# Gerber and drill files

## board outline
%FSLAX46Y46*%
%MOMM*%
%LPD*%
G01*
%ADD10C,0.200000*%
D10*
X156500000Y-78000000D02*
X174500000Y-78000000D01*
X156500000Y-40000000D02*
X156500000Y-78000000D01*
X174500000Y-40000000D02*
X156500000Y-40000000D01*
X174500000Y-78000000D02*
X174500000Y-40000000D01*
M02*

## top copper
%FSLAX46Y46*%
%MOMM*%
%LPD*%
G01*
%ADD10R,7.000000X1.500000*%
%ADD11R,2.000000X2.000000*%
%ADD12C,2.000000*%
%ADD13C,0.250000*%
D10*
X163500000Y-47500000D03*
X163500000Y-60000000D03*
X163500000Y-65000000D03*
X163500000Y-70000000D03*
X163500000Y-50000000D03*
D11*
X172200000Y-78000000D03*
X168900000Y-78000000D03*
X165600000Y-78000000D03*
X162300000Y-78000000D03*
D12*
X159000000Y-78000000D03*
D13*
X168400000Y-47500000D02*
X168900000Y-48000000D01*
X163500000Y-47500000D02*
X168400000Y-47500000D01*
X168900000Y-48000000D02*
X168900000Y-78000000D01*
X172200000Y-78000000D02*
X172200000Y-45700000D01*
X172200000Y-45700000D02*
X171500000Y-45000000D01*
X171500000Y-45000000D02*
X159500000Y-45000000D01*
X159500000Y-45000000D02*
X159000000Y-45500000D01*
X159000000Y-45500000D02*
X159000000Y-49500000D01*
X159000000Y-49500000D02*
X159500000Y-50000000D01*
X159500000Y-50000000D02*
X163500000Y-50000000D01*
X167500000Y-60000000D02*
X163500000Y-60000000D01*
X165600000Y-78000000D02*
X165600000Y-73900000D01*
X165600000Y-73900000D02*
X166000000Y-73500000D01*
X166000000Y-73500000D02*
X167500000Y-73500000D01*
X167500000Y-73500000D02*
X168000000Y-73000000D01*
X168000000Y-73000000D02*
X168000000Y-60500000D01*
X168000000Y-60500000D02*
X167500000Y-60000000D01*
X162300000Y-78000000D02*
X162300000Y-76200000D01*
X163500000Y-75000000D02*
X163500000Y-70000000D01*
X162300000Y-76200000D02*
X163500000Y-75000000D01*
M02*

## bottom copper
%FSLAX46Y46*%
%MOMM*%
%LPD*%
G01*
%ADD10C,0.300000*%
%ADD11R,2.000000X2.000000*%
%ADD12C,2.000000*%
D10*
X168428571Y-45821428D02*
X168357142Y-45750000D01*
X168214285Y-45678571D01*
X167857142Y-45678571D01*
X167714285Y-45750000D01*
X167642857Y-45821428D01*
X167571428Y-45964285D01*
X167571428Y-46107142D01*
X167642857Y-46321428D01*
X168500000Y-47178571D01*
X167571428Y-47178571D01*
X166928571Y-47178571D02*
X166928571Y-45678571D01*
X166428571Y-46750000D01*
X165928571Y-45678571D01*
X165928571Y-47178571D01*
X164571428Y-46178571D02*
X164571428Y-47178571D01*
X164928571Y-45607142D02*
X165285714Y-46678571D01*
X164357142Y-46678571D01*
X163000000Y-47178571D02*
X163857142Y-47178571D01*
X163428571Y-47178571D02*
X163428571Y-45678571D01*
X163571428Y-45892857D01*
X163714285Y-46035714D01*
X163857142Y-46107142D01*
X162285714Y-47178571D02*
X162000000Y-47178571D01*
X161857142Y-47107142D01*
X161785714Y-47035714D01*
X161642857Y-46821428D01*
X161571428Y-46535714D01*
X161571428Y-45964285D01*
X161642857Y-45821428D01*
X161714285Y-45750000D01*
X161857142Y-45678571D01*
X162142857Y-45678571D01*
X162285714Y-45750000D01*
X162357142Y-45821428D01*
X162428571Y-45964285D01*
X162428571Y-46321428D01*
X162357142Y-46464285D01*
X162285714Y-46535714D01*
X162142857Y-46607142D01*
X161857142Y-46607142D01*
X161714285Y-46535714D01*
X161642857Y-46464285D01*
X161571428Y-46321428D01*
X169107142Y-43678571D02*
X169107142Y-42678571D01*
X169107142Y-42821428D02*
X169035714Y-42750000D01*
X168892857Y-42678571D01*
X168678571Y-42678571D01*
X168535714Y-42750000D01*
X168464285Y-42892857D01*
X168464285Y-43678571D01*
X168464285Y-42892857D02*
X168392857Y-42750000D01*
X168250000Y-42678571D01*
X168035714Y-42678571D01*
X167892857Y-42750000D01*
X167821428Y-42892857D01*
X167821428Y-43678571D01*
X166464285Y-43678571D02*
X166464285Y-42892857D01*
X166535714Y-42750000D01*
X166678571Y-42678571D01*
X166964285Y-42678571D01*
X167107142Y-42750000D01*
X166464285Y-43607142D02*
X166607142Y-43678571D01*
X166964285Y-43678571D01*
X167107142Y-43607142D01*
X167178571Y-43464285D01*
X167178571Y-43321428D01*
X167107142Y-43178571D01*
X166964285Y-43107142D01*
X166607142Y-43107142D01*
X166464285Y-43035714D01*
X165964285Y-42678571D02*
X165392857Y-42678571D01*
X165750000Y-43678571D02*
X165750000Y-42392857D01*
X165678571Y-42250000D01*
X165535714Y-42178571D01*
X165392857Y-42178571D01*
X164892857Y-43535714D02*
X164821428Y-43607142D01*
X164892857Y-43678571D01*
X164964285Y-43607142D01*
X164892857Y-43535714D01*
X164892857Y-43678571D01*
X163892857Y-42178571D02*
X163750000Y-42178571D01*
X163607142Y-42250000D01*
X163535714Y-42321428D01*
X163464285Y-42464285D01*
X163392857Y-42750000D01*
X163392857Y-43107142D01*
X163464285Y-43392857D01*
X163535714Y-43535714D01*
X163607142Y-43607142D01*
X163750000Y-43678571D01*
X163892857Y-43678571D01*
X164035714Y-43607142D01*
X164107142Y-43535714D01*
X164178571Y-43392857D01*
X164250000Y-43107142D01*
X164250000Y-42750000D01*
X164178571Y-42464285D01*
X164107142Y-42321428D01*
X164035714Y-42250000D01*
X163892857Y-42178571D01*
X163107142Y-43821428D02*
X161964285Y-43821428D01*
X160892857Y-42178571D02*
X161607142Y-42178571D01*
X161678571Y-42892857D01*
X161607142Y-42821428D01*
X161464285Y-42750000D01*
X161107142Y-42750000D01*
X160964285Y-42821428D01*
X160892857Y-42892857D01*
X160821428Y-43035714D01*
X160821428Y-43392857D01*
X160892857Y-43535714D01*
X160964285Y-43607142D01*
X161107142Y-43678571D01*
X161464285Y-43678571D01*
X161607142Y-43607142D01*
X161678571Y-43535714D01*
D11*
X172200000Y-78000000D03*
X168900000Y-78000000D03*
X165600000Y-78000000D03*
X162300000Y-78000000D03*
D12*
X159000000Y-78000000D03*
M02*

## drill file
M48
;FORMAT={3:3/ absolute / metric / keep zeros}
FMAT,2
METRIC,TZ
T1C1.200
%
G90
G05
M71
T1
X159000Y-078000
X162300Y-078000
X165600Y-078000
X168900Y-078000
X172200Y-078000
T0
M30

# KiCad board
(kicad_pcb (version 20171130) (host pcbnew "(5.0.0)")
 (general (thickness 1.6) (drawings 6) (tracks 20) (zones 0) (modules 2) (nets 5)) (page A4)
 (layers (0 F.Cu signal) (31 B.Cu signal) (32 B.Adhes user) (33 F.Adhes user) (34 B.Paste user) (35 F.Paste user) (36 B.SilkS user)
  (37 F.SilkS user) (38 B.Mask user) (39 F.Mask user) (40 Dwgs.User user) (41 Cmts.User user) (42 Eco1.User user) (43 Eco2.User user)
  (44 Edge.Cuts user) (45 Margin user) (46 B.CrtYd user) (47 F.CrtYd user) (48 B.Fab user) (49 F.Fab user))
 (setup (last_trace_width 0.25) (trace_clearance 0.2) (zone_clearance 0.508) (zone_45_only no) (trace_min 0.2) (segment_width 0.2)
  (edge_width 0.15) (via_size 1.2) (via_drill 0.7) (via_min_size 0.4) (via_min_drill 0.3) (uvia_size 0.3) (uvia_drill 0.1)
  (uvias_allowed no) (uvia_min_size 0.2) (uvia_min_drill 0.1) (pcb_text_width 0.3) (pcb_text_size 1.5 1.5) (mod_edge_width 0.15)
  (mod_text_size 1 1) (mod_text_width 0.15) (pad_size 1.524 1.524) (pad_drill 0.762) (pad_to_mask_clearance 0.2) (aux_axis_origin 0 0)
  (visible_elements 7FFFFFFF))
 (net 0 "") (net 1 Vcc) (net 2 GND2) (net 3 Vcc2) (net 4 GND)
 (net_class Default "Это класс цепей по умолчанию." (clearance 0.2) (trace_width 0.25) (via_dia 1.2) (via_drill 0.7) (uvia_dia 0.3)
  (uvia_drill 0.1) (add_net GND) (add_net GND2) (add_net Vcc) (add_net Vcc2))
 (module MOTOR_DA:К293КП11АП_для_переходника (layer F.Cu) (at 163.5 86.5)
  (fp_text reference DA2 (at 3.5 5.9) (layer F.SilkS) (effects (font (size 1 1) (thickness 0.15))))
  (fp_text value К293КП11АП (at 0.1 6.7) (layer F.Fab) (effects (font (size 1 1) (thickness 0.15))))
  (pad 11 smd rect (at 0 -39) (size 7 1.5) (layers F.Cu F.Paste F.Mask) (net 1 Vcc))
  (pad 6 smd rect (at 0 -26.5) (size 7 1.5) (layers F.Cu F.Paste F.Mask) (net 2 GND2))
  (pad 4 smd rect (at 0 -21.5) (size 7 1.5) (layers F.Cu F.Paste F.Mask))
  (pad 2 smd rect (at 0 -16.5) (size 7 1.5) (layers F.Cu F.Paste F.Mask) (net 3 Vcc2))
  (pad 10 smd rect (at 0 -36.5) (size 7 1.5) (layers F.Cu F.Paste F.Mask) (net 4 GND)))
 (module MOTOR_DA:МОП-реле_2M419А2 (layer F.Cu) (at 159 78)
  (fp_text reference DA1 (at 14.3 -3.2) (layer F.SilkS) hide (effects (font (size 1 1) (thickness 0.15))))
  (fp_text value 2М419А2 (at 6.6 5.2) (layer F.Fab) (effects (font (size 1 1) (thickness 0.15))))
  (pad 5 thru_hole rect (at 13.2 0) (size 2 2) (drill 1.2) (layers *.Cu *.Paste *.Mask) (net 4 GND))
  (pad 4 thru_hole rect (at 9.9 0) (size 2 2) (drill 1.2) (layers *.Cu *.Paste *.Mask) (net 1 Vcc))
  (pad 3 thru_hole rect (at 6.6 0) (size 2 2) (drill 1.2) (layers *.Cu *.Paste *.Mask) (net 2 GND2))
  (pad 2 thru_hole rect (at 3.3 0) (size 2 2) (drill 1.2) (layers *.Cu *.Paste *.Mask) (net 3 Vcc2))
  (pad 1 thru_hole circle (at 0 0) (size 2 2) (drill 1.2) (layers *.Cu *.Paste *.Mask)))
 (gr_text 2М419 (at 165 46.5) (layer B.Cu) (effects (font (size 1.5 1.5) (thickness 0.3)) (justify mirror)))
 (gr_line (start 156.5 78) (end 174.5 78) (layer Edge.Cuts) (width 0.2))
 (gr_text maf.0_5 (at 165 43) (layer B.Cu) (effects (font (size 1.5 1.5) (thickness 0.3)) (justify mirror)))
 (gr_line (start 156.5 40) (end 156.5 78) (layer Edge.Cuts) (width 0.2))
 (gr_line (start 174.5 40) (end 156.5 40) (layer Edge.Cuts) (width 0.2))
 (gr_line (start 174.5 78) (end 174.5 40) (layer Edge.Cuts) (width 0.2))
 (segment (start 168.4 47.5) (end 168.9 48) (width 0.25) (layer F.Cu) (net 1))
 (segment (start 163.5 47.5) (end 168.4 47.5) (width 0.25) (layer F.Cu) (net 1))
 (segment (start 168.9 48) (end 168.9 78) (width 0.25) (layer F.Cu) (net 1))
 (segment (start 172.2 78) (end 172.2 45.7) (width 0.25) (layer F.Cu) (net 4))
 (segment (start 172.2 45.7) (end 171.5 45) (width 0.25) (layer F.Cu) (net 4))
 (segment (start 171.5 45) (end 159.5 45) (width 0.25) (layer F.Cu) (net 4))
 (segment (start 159.5 45) (end 159 45.5) (width 0.25) (layer F.Cu) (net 4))
 (segment (start 159 45.5) (end 159 49.5) (width 0.25) (layer F.Cu) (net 4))
 (segment (start 159 49.5) (end 159.5 50) (width 0.25) (layer F.Cu) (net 4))
 (segment (start 159.5 50) (end 163.5 50) (width 0.25) (layer F.Cu) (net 4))
 (segment (start 167.5 60) (end 163.5 60) (width 0.25) (layer F.Cu) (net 2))
 (segment (start 165.6 78) (end 165.6 73.9) (width 0.25) (layer F.Cu) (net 2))
 (segment (start 165.6 73.9) (end 166 73.5) (width 0.25) (layer F.Cu) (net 2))
 (segment (start 166 73.5) (end 167.5 73.5) (width 0.25) (layer F.Cu) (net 2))
 (segment (start 167.5 73.5) (end 168 73) (width 0.25) (layer F.Cu) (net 2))
 (segment (start 168 73) (end 168 60.5) (width 0.25) (layer F.Cu) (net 2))
 (segment (start 168 60.5) (end 167.5 60) (width 0.25) (layer F.Cu) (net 2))
 (segment (start 162.3 78) (end 162.3 76.2) (width 0.25) (layer F.Cu) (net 3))
 (segment (start 163.5 75) (end 163.5 70) (width 0.25) (layer F.Cu) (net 3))
 (segment (start 162.3 76.2) (end 163.5 75) (width 0.25) (layer F.Cu) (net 3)))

